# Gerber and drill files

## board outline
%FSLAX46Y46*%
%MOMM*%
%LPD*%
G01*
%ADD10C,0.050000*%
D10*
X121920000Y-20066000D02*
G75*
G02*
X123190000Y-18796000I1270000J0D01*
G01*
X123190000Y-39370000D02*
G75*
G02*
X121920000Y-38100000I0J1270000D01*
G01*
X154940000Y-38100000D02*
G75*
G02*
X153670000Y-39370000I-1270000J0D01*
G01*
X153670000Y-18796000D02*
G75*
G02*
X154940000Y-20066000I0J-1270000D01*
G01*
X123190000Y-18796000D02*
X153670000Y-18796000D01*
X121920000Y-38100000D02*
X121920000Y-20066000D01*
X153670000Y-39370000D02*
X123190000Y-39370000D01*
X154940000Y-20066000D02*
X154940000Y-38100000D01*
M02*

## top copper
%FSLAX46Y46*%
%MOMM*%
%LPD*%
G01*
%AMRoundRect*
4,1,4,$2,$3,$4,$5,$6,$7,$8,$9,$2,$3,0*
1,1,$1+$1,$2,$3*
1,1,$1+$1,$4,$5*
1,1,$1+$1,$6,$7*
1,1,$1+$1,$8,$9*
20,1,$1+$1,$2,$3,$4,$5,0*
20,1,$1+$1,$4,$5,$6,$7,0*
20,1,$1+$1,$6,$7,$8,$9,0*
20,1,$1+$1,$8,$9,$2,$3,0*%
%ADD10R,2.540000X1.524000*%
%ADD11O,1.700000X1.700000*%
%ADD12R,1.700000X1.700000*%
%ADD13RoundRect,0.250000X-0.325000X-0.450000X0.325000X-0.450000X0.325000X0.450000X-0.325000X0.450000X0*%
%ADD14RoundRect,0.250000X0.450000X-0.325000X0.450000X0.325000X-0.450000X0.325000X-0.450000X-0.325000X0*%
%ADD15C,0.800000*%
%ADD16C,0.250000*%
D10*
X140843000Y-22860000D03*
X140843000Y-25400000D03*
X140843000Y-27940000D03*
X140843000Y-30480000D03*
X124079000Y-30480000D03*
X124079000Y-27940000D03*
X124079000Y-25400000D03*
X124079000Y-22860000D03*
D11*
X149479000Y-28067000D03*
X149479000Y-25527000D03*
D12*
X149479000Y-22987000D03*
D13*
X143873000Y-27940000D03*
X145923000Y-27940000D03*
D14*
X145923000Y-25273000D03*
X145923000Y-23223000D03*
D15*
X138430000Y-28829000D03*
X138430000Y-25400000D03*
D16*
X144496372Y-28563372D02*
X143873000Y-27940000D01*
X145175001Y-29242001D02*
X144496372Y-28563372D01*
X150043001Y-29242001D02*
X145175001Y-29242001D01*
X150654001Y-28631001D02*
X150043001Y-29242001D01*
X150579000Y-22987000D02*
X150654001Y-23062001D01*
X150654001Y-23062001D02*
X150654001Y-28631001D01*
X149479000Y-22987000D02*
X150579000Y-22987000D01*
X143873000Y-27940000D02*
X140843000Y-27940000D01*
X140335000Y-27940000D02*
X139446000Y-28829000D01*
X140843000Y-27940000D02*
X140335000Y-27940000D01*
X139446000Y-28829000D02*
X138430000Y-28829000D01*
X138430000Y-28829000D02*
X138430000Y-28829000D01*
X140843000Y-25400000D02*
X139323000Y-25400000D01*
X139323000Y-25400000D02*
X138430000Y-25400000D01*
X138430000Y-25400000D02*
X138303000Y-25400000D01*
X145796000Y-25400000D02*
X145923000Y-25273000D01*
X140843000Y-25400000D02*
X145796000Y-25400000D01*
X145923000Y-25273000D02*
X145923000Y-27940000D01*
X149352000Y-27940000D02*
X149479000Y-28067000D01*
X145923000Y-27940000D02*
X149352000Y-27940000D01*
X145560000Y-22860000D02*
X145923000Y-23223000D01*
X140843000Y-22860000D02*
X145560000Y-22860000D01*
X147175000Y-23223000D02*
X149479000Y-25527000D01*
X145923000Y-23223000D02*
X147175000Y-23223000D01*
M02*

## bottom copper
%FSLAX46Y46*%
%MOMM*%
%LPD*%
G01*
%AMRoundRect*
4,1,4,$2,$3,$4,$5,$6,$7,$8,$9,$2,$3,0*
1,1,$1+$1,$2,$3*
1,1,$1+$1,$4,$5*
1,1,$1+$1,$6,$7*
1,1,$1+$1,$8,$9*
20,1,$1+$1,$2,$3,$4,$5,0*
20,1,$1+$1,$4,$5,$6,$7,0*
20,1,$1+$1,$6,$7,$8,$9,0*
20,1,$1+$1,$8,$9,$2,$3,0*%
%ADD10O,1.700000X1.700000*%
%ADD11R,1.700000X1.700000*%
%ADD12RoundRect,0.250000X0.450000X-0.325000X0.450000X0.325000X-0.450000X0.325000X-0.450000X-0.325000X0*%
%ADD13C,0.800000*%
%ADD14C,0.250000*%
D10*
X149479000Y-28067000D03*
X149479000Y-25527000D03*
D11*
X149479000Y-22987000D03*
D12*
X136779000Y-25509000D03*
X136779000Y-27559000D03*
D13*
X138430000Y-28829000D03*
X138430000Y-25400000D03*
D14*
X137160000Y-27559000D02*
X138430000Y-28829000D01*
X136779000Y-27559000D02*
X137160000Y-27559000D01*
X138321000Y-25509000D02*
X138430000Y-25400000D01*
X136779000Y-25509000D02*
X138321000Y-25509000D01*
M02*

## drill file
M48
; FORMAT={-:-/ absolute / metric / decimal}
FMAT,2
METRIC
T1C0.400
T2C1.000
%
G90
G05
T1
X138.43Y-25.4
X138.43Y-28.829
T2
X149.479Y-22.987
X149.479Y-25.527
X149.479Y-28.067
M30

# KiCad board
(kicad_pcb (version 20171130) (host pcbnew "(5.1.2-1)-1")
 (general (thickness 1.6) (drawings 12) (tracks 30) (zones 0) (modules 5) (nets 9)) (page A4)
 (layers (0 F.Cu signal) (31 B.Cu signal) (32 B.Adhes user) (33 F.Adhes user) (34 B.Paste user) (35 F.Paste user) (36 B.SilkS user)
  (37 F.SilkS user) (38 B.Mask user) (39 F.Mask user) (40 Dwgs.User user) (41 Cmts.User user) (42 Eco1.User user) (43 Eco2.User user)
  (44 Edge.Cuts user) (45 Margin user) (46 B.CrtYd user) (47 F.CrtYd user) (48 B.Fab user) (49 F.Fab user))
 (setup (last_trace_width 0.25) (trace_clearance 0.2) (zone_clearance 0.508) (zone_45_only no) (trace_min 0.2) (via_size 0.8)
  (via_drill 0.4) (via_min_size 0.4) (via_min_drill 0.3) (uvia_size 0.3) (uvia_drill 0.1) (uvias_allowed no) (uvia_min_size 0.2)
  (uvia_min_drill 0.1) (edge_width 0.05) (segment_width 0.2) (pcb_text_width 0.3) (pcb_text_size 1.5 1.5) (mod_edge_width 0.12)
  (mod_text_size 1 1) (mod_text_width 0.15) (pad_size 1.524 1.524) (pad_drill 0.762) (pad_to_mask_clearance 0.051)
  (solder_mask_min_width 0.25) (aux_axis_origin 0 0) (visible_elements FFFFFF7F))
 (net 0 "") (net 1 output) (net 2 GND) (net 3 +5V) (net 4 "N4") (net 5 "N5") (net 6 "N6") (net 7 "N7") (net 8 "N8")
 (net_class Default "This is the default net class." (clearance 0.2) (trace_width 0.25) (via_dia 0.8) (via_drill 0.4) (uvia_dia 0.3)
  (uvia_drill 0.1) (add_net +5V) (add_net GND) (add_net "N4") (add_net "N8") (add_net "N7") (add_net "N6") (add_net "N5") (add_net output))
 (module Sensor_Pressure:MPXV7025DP (layer F.Cu) (at 132.461 26.67)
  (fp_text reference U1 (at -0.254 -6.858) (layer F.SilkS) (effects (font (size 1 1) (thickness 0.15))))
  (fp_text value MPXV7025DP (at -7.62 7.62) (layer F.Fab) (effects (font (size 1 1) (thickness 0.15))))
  (pad 4 smd rect (at 8.382 -3.81) (size 2.54 1.524) (layers F.Cu F.Paste F.Mask) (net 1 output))
  (pad 3 smd rect (at 8.382 -1.27) (size 2.54 1.524) (layers F.Cu F.Paste F.Mask) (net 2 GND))
  (pad 2 smd rect (at 8.382 1.27) (size 2.54 1.524) (layers F.Cu F.Paste F.Mask) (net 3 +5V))
  (pad 1 smd rect (at 8.382 3.81) (size 2.54 1.524) (layers F.Cu F.Paste F.Mask) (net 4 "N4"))
  (pad 8 smd rect (at -8.382 3.81) (size 2.54 1.524) (layers F.Cu F.Paste F.Mask) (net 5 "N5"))
  (pad 7 smd rect (at -8.382 1.27) (size 2.54 1.524) (layers F.Cu F.Paste F.Mask) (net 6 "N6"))
  (pad 6 smd rect (at -8.382 -1.27) (size 2.54 1.524) (layers F.Cu F.Paste F.Mask) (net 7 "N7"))
  (pad 5 smd rect (at -8.382 -3.81) (size 2.54 1.524) (layers F.Cu F.Paste F.Mask) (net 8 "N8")))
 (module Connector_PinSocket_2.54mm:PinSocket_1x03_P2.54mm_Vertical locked (layer F.Cu) (at 149.479 22.987)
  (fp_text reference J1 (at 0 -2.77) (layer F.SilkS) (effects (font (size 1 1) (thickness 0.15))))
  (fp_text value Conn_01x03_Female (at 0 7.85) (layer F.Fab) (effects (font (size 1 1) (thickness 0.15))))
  (pad 3 thru_hole oval (at 0 5.08) (size 1.7 1.7) (drill 1) (layers *.Cu *.Mask) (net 2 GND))
  (pad 2 thru_hole oval (at 0 2.54) (size 1.7 1.7) (drill 1) (layers *.Cu *.Mask) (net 1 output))
  (pad 1 thru_hole rect (at 0 0) (size 1.7 1.7) (drill 1) (layers *.Cu *.Mask) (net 3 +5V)))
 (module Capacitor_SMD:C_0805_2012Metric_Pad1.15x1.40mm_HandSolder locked (layer F.Cu) (at 144.898 27.94)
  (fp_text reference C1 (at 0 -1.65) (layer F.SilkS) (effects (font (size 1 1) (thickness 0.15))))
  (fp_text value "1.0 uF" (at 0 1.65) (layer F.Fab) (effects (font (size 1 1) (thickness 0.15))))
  (pad 1 smd roundrect (at -1.025 0) (size 1.15 1.4) (layers F.Cu F.Paste F.Mask) (roundrect_rratio 0.217391) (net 3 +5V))
  (pad 2 smd roundrect (at 1.025 0) (size 1.15 1.4) (layers F.Cu F.Paste F.Mask) (roundrect_rratio 0.217391) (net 2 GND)))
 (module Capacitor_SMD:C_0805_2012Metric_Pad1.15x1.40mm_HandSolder (layer B.Cu) (at 136.779 26.534 90)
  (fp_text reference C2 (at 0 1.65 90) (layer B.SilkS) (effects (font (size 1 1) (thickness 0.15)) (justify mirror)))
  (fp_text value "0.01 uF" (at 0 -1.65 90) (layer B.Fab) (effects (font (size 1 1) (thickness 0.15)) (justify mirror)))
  (pad 2 smd roundrect (at 1.025 0 90) (size 1.15 1.4) (layers B.Cu B.Paste B.Mask) (roundrect_rratio 0.217391) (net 2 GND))
  (pad 1 smd roundrect (at -1.025 0 90) (size 1.15 1.4) (layers B.Cu B.Paste B.Mask) (roundrect_rratio 0.217391) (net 3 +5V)))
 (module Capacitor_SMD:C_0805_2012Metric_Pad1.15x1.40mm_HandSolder (layer F.Cu) (at 145.923 24.248 90)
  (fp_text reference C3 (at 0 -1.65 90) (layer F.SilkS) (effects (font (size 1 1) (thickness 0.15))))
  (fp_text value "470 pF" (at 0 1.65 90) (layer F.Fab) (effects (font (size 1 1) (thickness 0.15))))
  (pad 1 smd roundrect (at -1.025 0 90) (size 1.15 1.4) (layers F.Cu F.Paste F.Mask) (roundrect_rratio 0.217391) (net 2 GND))
  (pad 2 smd roundrect (at 1.025 0 90) (size 1.15 1.4) (layers F.Cu F.Paste F.Mask) (roundrect_rratio 0.217391) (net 1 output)))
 (gr_arc (start 123.19 20.066) (end 123.19 18.796) (angle -90) (layer Edge.Cuts) (width 0.05))
 (gr_arc (start 123.19 38.1) (end 121.92 38.1) (angle -90) (layer Edge.Cuts) (width 0.05))
 (gr_arc (start 153.67 38.1) (end 153.67 39.37) (angle -90) (layer Edge.Cuts) (width 0.05))
 (gr_arc (start 153.67 20.066) (end 154.94 20.066) (angle -90) (layer Edge.Cuts) (width 0.05))
 (gr_line (start 123.19 18.796) (end 153.67 18.796) (layer Edge.Cuts) (width 0.05))
 (gr_line (start 121.92 38.1) (end 121.92 20.066) (layer Edge.Cuts) (width 0.05))
 (gr_line (start 153.67 39.37) (end 123.19 39.37) (layer Edge.Cuts) (width 0.05))
 (gr_line (start 154.94 20.066) (end 154.94 38.1) (layer Edge.Cuts) (width 0.05))
 (segment (start 144.496372 28.563372) (end 143.873 27.94) (width 0.25) (layer F.Cu) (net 3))
 (segment (start 145.175001 29.242001) (end 144.496372 28.563372) (width 0.25) (layer F.Cu) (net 3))
 (segment (start 150.043001 29.242001) (end 145.175001 29.242001) (width 0.25) (layer F.Cu) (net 3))
 (segment (start 150.654001 28.631001) (end 150.043001 29.242001) (width 0.25) (layer F.Cu) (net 3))
 (segment (start 150.579 22.987) (end 150.654001 23.062001) (width 0.25) (layer F.Cu) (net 3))
 (segment (start 150.654001 23.062001) (end 150.654001 28.631001) (width 0.25) (layer F.Cu) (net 3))
 (segment (start 149.479 22.987) (end 150.579 22.987) (width 0.25) (layer F.Cu) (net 3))
 (segment (start 143.873 27.94) (end 140.843 27.94) (width 0.25) (layer F.Cu) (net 3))
 (segment (start 140.335 27.94) (end 139.446 28.829) (width 0.25) (layer F.Cu) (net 3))
 (segment (start 140.843 27.94) (end 140.335 27.94) (width 0.25) (layer F.Cu) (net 3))
 (segment (start 139.446 28.829) (end 138.43 28.829) (width 0.25) (layer F.Cu) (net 3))
 (segment (start 138.43 28.829) (end 138.43 28.829) (width 0.25) (layer F.Cu) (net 3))
 (via (at 138.43 28.829) (size 0.8) (drill 0.4) (layers F.Cu B.Cu) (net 3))
 (segment (start 137.16 27.559) (end 138.43 28.829) (width 0.25) (layer B.Cu) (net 3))
 (segment (start 136.779 27.559) (end 137.16 27.559) (width 0.25) (layer B.Cu) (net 3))
 (segment (start 140.843 25.4) (end 139.323 25.4) (width 0.25) (layer F.Cu) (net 2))
 (segment (start 139.323 25.4) (end 138.43 25.4) (width 0.25) (layer F.Cu) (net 2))
 (segment (start 138.43 25.4) (end 138.303 25.4) (width 0.25) (layer F.Cu) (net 2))
 (via (at 138.43 25.4) (size 0.8) (drill 0.4) (layers F.Cu B.Cu) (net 2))
 (segment (start 138.321 25.509) (end 138.43 25.4) (width 0.25) (layer B.Cu) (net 2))
 (segment (start 136.779 25.509) (end 138.321 25.509) (width 0.25) (layer B.Cu) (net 2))
 (segment (start 145.796 25.4) (end 145.923 25.273) (width 0.25) (layer F.Cu) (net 2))
 (segment (start 140.843 25.4) (end 145.796 25.4) (width 0.25) (layer F.Cu) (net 2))
 (segment (start 145.923 25.273) (end 145.923 27.94) (width 0.25) (layer F.Cu) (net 2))
 (segment (start 149.352 27.94) (end 149.479 28.067) (width 0.25) (layer F.Cu) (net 2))
 (segment (start 145.923 27.94) (end 149.352 27.94) (width 0.25) (layer F.Cu) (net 2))
 (segment (start 145.56 22.86) (end 145.923 23.223) (width 0.25) (layer F.Cu) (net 1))
 (segment (start 140.843 22.86) (end 145.56 22.86) (width 0.25) (layer F.Cu) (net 1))
 (segment (start 147.175 23.223) (end 149.479 25.527) (width 0.25) (layer F.Cu) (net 1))
 (segment (start 145.923 23.223) (end 147.175 23.223) (width 0.25) (layer F.Cu) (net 1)))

